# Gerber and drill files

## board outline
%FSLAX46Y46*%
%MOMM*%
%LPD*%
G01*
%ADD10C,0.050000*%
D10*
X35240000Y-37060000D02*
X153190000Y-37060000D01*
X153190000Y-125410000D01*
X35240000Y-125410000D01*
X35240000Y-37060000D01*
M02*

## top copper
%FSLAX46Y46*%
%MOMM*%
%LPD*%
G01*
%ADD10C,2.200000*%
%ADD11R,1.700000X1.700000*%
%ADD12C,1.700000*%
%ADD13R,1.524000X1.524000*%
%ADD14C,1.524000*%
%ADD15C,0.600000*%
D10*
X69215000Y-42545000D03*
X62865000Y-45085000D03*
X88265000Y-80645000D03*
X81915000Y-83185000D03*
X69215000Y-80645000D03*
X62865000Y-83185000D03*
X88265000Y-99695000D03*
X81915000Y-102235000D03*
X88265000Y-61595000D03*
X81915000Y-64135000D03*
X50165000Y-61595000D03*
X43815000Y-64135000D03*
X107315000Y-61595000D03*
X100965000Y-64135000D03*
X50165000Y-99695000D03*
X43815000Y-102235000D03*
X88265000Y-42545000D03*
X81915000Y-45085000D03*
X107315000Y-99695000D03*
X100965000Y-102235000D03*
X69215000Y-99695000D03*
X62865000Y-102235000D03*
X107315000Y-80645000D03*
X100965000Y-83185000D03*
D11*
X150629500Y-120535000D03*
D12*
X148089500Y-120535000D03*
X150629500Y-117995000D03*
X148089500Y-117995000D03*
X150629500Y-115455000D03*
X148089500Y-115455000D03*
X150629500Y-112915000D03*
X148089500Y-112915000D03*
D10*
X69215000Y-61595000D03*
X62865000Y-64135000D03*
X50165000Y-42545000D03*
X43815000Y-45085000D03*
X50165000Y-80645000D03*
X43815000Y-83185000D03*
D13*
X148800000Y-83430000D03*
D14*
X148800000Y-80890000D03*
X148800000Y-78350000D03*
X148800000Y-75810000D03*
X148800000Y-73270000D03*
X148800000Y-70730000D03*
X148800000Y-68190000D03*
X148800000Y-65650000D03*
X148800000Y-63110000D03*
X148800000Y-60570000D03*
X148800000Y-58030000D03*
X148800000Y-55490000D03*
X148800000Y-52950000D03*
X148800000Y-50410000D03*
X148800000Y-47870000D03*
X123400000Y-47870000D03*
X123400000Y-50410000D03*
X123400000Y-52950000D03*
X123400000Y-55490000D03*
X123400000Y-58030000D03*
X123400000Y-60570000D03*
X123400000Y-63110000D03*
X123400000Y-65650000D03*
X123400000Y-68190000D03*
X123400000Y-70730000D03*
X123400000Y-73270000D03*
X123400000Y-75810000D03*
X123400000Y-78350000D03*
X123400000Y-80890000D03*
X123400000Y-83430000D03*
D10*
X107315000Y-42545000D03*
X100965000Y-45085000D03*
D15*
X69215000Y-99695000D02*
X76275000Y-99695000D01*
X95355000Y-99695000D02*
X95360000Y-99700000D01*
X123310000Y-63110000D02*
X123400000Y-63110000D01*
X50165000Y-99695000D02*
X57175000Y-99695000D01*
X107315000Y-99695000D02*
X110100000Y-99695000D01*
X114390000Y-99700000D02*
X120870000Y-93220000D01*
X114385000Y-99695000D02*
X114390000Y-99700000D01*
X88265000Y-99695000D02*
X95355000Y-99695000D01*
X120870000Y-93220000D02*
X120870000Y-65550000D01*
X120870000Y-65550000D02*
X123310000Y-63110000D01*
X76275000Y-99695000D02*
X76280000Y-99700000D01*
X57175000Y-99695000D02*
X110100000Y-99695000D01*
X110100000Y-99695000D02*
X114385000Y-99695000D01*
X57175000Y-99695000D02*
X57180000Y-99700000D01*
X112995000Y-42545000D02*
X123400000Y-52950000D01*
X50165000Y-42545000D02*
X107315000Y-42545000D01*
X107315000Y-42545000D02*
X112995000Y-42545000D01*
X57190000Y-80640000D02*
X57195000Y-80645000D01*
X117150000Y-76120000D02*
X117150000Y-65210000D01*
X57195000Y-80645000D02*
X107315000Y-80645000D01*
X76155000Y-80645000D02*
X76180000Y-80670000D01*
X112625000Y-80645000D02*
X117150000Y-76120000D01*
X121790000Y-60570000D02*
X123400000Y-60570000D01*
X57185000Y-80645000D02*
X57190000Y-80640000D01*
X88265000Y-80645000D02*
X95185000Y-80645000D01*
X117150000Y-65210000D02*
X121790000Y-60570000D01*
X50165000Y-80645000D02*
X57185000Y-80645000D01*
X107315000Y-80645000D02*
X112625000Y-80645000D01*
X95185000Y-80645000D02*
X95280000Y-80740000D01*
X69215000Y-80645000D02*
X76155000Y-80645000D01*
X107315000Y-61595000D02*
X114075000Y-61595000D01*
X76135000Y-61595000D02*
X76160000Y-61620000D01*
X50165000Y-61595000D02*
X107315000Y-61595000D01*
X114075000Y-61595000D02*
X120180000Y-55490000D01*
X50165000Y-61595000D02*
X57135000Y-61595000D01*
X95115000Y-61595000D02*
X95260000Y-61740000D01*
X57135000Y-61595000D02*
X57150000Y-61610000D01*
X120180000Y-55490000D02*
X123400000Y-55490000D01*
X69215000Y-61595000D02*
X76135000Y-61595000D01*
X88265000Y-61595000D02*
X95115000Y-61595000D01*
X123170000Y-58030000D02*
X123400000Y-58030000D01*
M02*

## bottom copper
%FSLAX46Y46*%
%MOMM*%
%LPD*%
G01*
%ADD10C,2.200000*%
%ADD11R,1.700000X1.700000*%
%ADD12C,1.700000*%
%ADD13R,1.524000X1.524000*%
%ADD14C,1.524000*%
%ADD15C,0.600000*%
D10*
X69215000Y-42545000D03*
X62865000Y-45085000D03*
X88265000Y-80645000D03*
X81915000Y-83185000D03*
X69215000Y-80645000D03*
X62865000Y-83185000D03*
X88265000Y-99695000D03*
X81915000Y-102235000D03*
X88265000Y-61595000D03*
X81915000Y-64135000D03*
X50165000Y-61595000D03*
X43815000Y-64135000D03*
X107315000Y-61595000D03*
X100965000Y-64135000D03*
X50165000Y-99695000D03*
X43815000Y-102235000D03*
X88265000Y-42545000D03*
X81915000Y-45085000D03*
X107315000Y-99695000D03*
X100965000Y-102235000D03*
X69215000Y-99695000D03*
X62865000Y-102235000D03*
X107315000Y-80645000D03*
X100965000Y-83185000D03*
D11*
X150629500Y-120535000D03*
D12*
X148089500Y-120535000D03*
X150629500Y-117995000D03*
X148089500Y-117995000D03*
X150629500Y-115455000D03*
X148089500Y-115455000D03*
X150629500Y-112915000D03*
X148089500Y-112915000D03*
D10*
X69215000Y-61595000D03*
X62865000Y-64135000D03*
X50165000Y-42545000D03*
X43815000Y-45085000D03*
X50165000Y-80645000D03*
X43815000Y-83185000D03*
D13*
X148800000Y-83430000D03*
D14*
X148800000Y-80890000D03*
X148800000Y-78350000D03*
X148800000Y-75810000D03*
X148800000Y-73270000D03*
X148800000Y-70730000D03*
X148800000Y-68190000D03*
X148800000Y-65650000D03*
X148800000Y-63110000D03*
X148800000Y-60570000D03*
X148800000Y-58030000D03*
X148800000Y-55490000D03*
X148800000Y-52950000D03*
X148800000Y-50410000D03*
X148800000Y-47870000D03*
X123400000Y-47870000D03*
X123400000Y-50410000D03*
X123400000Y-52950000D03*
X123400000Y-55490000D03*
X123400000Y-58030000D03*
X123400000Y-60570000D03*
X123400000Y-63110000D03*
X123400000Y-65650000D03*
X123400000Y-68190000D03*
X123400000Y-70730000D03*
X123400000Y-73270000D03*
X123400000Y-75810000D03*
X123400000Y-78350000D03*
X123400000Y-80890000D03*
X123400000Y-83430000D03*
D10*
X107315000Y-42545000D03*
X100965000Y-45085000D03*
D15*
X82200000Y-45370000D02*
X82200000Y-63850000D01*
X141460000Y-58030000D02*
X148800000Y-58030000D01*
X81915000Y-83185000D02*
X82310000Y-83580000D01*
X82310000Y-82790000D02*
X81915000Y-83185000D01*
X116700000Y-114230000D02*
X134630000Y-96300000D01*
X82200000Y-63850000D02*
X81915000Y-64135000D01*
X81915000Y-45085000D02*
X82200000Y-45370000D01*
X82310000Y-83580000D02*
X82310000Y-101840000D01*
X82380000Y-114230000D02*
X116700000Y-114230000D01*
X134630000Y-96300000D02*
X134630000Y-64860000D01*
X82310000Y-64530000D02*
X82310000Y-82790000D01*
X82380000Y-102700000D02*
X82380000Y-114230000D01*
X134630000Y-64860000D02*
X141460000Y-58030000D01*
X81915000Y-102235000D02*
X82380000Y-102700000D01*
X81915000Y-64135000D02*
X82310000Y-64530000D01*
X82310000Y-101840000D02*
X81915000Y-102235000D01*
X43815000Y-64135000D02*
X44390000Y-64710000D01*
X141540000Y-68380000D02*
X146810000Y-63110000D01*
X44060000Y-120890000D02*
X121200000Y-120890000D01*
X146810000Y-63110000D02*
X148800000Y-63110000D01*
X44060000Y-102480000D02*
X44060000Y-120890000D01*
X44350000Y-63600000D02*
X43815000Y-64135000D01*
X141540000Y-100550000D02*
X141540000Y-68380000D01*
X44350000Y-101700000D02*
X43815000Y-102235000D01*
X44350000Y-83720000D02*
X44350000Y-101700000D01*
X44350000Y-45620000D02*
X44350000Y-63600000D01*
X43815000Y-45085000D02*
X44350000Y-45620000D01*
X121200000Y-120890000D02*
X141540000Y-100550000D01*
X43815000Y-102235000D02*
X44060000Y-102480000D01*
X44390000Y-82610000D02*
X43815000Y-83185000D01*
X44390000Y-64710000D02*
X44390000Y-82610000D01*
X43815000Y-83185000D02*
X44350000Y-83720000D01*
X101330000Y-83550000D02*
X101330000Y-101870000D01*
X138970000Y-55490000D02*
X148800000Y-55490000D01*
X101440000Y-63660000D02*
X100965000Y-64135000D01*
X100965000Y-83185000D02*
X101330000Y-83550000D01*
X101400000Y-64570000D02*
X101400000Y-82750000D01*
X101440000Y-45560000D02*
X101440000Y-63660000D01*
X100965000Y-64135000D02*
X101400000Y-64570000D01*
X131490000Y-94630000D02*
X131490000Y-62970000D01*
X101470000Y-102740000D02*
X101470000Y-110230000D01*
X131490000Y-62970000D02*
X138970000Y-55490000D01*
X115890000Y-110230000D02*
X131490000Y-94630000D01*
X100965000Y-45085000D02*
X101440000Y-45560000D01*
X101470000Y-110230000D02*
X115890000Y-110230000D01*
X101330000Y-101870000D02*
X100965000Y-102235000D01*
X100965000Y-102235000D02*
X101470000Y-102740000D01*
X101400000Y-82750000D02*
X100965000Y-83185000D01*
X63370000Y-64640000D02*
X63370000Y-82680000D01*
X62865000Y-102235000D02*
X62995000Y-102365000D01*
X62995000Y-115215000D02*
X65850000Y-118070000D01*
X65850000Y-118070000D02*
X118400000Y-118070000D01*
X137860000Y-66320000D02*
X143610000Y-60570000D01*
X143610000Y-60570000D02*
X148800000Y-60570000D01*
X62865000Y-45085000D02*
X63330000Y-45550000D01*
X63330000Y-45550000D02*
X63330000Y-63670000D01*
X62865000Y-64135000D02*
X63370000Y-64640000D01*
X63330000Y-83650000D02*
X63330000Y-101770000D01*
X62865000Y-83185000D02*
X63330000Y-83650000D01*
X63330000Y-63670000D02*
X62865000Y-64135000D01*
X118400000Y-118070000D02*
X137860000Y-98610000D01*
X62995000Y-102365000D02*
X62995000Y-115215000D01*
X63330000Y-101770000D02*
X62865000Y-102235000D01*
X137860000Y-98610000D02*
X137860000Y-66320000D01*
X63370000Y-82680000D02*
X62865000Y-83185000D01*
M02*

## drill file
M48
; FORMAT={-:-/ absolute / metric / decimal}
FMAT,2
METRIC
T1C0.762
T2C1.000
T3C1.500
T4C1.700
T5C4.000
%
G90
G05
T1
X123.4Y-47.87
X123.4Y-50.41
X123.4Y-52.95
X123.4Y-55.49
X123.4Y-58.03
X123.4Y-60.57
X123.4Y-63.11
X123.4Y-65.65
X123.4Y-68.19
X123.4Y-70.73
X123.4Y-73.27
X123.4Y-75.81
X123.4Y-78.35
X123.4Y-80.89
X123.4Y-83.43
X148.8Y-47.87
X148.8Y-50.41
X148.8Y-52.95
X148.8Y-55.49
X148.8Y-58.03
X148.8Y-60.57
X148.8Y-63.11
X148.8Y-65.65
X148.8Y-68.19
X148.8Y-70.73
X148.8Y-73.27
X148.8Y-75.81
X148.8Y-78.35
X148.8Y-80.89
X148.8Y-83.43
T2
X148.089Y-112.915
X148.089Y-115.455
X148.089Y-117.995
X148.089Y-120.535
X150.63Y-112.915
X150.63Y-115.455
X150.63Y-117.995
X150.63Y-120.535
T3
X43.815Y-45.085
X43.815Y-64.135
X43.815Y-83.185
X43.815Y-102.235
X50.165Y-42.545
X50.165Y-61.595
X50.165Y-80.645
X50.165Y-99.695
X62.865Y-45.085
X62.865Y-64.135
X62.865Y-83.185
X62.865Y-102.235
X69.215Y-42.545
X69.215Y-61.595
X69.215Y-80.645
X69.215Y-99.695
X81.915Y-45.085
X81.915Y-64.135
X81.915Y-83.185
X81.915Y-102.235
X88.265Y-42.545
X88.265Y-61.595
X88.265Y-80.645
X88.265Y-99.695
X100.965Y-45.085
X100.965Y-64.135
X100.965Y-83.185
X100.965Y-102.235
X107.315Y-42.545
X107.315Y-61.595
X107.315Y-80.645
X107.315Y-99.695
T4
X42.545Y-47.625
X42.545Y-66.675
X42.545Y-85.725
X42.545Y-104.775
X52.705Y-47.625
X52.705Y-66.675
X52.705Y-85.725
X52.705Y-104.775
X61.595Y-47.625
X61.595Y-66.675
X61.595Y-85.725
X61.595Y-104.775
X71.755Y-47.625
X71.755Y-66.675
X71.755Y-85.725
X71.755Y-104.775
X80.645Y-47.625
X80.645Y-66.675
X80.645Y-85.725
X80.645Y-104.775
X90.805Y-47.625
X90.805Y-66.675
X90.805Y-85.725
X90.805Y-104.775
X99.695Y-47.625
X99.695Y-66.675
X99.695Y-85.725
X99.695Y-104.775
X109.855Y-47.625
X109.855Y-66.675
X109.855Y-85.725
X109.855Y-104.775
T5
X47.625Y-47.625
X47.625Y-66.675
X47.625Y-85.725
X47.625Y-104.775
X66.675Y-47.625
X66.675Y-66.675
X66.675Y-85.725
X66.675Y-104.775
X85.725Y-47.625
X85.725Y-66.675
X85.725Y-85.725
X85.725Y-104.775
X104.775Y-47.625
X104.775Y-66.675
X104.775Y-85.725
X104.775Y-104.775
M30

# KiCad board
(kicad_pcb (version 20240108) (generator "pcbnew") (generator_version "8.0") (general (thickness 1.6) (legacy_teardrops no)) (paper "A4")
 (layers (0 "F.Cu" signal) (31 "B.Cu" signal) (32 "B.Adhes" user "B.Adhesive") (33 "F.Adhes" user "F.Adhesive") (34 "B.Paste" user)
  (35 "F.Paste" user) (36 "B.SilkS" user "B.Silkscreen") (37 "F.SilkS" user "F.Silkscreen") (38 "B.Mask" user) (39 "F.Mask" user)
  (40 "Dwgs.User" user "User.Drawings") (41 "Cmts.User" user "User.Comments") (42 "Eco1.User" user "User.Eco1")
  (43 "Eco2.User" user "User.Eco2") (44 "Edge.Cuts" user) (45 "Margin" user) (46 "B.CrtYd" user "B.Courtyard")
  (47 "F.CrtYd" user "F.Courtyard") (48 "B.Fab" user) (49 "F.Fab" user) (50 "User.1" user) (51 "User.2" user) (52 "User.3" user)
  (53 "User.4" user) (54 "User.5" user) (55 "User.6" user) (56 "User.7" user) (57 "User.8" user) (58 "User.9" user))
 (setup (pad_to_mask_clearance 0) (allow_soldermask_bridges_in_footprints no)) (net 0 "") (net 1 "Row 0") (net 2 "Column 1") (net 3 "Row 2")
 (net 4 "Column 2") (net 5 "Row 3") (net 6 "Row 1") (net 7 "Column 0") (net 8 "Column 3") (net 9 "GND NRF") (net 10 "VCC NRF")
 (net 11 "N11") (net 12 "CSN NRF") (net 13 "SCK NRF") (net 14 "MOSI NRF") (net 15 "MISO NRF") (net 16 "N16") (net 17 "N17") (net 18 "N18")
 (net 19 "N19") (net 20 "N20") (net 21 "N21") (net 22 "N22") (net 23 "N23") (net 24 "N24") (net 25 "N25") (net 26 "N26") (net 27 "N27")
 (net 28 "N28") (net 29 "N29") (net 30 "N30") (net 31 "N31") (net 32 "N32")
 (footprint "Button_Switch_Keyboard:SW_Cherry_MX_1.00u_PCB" (layer "F.Cu") (at 69.215 42.545)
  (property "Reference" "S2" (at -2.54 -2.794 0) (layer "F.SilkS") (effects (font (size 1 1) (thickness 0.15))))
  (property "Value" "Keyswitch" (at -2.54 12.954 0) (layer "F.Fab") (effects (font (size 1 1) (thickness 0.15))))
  (pad "" np_thru_hole circle (at -7.62 5.08) (size 1.7 1.7) (drill 1.7) (layers "*.Cu" "*.Mask"))
  (pad "" np_thru_hole circle (at -2.54 5.08) (size 4 4) (drill 4) (layers "*.Cu" "*.Mask"))
  (pad "" np_thru_hole circle (at 2.54 5.08) (size 1.7 1.7) (drill 1.7) (layers "*.Cu" "*.Mask"))
  (pad "1" thru_hole circle (at 0 0) (size 2.2 2.2) (drill 1.5) (layers "*.Cu" "*.Mask") (remove_unused_layers no) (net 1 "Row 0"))
  (pad "2" thru_hole circle (at -6.35 2.54) (size 2.2 2.2) (drill 1.5) (layers "*.Cu" "*.Mask") (remove_unused_layers no) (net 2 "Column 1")))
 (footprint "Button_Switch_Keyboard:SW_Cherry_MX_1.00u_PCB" (layer "F.Cu") (at 88.265 80.645)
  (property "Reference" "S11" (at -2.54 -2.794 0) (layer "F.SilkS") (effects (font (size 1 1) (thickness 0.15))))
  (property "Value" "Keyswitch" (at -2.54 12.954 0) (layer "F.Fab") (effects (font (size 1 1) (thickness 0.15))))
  (pad "" np_thru_hole circle (at -7.62 5.08) (size 1.7 1.7) (drill 1.7) (layers "*.Cu" "*.Mask"))
  (pad "" np_thru_hole circle (at -2.54 5.08) (size 4 4) (drill 4) (layers "*.Cu" "*.Mask"))
  (pad "" np_thru_hole circle (at 2.54 5.08) (size 1.7 1.7) (drill 1.7) (layers "*.Cu" "*.Mask"))
  (pad "1" thru_hole circle (at 0 0) (size 2.2 2.2) (drill 1.5) (layers "*.Cu" "*.Mask") (remove_unused_layers no) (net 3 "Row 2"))
  (pad "2" thru_hole circle (at -6.35 2.54) (size 2.2 2.2) (drill 1.5) (layers "*.Cu" "*.Mask") (remove_unused_layers no) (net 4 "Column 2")))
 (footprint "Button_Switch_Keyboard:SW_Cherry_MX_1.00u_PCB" (layer "F.Cu") (at 69.215 80.645)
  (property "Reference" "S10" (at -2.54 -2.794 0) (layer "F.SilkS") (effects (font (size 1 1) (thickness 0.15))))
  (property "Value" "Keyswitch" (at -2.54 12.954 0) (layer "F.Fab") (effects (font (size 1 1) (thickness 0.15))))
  (pad "" np_thru_hole circle (at -7.62 5.08) (size 1.7 1.7) (drill 1.7) (layers "*.Cu" "*.Mask"))
  (pad "" np_thru_hole circle (at -2.54 5.08) (size 4 4) (drill 4) (layers "*.Cu" "*.Mask"))
  (pad "" np_thru_hole circle (at 2.54 5.08) (size 1.7 1.7) (drill 1.7) (layers "*.Cu" "*.Mask"))
  (pad "1" thru_hole circle (at 0 0) (size 2.2 2.2) (drill 1.5) (layers "*.Cu" "*.Mask") (remove_unused_layers no) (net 3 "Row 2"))
  (pad "2" thru_hole circle (at -6.35 2.54) (size 2.2 2.2) (drill 1.5) (layers "*.Cu" "*.Mask") (remove_unused_layers no) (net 2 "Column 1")))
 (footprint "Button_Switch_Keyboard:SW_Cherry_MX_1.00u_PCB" (layer "F.Cu") (at 88.265 99.695)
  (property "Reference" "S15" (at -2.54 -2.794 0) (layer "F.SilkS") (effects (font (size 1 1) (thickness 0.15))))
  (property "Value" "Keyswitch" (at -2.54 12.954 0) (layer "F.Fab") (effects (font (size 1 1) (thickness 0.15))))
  (pad "" np_thru_hole circle (at -7.62 5.08) (size 1.7 1.7) (drill 1.7) (layers "*.Cu" "*.Mask"))
  (pad "" np_thru_hole circle (at -2.54 5.08) (size 4 4) (drill 4) (layers "*.Cu" "*.Mask"))
  (pad "" np_thru_hole circle (at 2.54 5.08) (size 1.7 1.7) (drill 1.7) (layers "*.Cu" "*.Mask"))
  (pad "1" thru_hole circle (at 0 0) (size 2.2 2.2) (drill 1.5) (layers "*.Cu" "*.Mask") (remove_unused_layers no) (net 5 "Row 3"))
  (pad "2" thru_hole circle (at -6.35 2.54) (size 2.2 2.2) (drill 1.5) (layers "*.Cu" "*.Mask") (remove_unused_layers no) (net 4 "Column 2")))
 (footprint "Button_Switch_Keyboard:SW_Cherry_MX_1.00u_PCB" (layer "F.Cu") (at 88.265 61.595)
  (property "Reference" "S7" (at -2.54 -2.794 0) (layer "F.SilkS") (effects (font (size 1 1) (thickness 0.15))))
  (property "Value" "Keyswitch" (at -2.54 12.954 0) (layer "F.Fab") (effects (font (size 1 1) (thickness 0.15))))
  (pad "" np_thru_hole circle (at -7.62 5.08) (size 1.7 1.7) (drill 1.7) (layers "*.Cu" "*.Mask"))
  (pad "" np_thru_hole circle (at -2.54 5.08) (size 4 4) (drill 4) (layers "*.Cu" "*.Mask"))
  (pad "" np_thru_hole circle (at 2.54 5.08) (size 1.7 1.7) (drill 1.7) (layers "*.Cu" "*.Mask"))
  (pad "1" thru_hole circle (at 0 0) (size 2.2 2.2) (drill 1.5) (layers "*.Cu" "*.Mask") (remove_unused_layers no) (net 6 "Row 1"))
  (pad "2" thru_hole circle (at -6.35 2.54) (size 2.2 2.2) (drill 1.5) (layers "*.Cu" "*.Mask") (remove_unused_layers no) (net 4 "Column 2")))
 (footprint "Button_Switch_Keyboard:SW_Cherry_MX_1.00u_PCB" (layer "F.Cu") (at 50.165 61.595)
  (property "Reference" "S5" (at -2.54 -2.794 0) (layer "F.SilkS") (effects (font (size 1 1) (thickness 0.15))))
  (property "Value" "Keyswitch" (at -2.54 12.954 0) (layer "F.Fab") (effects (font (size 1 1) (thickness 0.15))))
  (pad "" np_thru_hole circle (at -7.62 5.08) (size 1.7 1.7) (drill 1.7) (layers "*.Cu" "*.Mask"))
  (pad "" np_thru_hole circle (at -2.54 5.08) (size 4 4) (drill 4) (layers "*.Cu" "*.Mask"))
  (pad "" np_thru_hole circle (at 2.54 5.08) (size 1.7 1.7) (drill 1.7) (layers "*.Cu" "*.Mask"))
  (pad "1" thru_hole circle (at 0 0) (size 2.2 2.2) (drill 1.5) (layers "*.Cu" "*.Mask") (remove_unused_layers no) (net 6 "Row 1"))
  (pad "2" thru_hole circle (at -6.35 2.54) (size 2.2 2.2) (drill 1.5) (layers "*.Cu" "*.Mask") (remove_unused_layers no) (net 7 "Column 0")))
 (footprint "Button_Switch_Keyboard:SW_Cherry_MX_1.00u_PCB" (layer "F.Cu") (at 107.315 61.595)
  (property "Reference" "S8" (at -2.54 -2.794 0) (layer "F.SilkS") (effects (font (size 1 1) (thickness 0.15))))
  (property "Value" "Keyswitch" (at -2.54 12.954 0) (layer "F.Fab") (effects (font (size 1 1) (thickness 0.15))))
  (pad "" np_thru_hole circle (at -7.62 5.08) (size 1.7 1.7) (drill 1.7) (layers "*.Cu" "*.Mask"))
  (pad "" np_thru_hole circle (at -2.54 5.08) (size 4 4) (drill 4) (layers "*.Cu" "*.Mask"))
  (pad "" np_thru_hole circle (at 2.54 5.08) (size 1.7 1.7) (drill 1.7) (layers "*.Cu" "*.Mask"))
  (pad "1" thru_hole circle (at 0 0) (size 2.2 2.2) (drill 1.5) (layers "*.Cu" "*.Mask") (remove_unused_layers no) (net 6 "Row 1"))
  (pad "2" thru_hole circle (at -6.35 2.54) (size 2.2 2.2) (drill 1.5) (layers "*.Cu" "*.Mask") (remove_unused_layers no) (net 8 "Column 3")))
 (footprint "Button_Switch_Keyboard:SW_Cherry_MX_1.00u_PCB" (layer "F.Cu") (at 50.165 99.695)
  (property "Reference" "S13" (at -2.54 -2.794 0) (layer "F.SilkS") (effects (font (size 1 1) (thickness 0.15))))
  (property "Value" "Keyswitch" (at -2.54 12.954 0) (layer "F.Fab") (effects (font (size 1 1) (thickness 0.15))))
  (pad "" np_thru_hole circle (at -7.62 5.08) (size 1.7 1.7) (drill 1.7) (layers "*.Cu" "*.Mask"))
  (pad "" np_thru_hole circle (at -2.54 5.08) (size 4 4) (drill 4) (layers "*.Cu" "*.Mask"))
  (pad "" np_thru_hole circle (at 2.54 5.08) (size 1.7 1.7) (drill 1.7) (layers "*.Cu" "*.Mask"))
  (pad "1" thru_hole circle (at 0 0) (size 2.2 2.2) (drill 1.5) (layers "*.Cu" "*.Mask") (remove_unused_layers no) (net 5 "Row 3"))
  (pad "2" thru_hole circle (at -6.35 2.54) (size 2.2 2.2) (drill 1.5) (layers "*.Cu" "*.Mask") (remove_unused_layers no) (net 7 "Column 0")))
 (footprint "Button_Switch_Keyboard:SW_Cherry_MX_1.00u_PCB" (layer "F.Cu") (at 88.265 42.545)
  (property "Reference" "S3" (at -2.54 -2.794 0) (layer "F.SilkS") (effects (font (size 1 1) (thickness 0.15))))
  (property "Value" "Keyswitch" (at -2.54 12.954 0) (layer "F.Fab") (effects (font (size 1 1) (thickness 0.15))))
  (pad "" np_thru_hole circle (at -7.62 5.08) (size 1.7 1.7) (drill 1.7) (layers "*.Cu" "*.Mask"))
  (pad "" np_thru_hole circle (at -2.54 5.08) (size 4 4) (drill 4) (layers "*.Cu" "*.Mask"))
  (pad "" np_thru_hole circle (at 2.54 5.08) (size 1.7 1.7) (drill 1.7) (layers "*.Cu" "*.Mask"))
  (pad "1" thru_hole circle (at 0 0) (size 2.2 2.2) (drill 1.5) (layers "*.Cu" "*.Mask") (remove_unused_layers no) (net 1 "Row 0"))
  (pad "2" thru_hole circle (at -6.35 2.54) (size 2.2 2.2) (drill 1.5) (layers "*.Cu" "*.Mask") (remove_unused_layers no) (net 4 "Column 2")))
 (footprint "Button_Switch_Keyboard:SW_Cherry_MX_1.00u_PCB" (layer "F.Cu") (at 107.315 99.695)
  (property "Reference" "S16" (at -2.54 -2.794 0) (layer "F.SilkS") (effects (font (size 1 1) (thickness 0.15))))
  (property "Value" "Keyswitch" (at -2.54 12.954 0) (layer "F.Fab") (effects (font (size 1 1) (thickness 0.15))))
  (pad "" np_thru_hole circle (at -7.62 5.08) (size 1.7 1.7) (drill 1.7) (layers "*.Cu" "*.Mask"))
  (pad "" np_thru_hole circle (at -2.54 5.08) (size 4 4) (drill 4) (layers "*.Cu" "*.Mask"))
  (pad "" np_thru_hole circle (at 2.54 5.08) (size 1.7 1.7) (drill 1.7) (layers "*.Cu" "*.Mask"))
  (pad "1" thru_hole circle (at 0 0) (size 2.2 2.2) (drill 1.5) (layers "*.Cu" "*.Mask") (remove_unused_layers no) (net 5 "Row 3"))
  (pad "2" thru_hole circle (at -6.35 2.54) (size 2.2 2.2) (drill 1.5) (layers "*.Cu" "*.Mask") (remove_unused_layers no) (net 8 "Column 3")))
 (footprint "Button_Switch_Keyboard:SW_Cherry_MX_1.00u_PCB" (layer "F.Cu") (at 69.215 99.695)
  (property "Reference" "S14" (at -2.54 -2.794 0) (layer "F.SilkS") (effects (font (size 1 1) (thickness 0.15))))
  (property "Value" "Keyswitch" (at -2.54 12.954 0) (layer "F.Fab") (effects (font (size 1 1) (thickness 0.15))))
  (pad "" np_thru_hole circle (at -7.62 5.08) (size 1.7 1.7) (drill 1.7) (layers "*.Cu" "*.Mask"))
  (pad "" np_thru_hole circle (at -2.54 5.08) (size 4 4) (drill 4) (layers "*.Cu" "*.Mask"))
  (pad "" np_thru_hole circle (at 2.54 5.08) (size 1.7 1.7) (drill 1.7) (layers "*.Cu" "*.Mask"))
  (pad "1" thru_hole circle (at 0 0) (size 2.2 2.2) (drill 1.5) (layers "*.Cu" "*.Mask") (remove_unused_layers no) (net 5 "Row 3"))
  (pad "2" thru_hole circle (at -6.35 2.54) (size 2.2 2.2) (drill 1.5) (layers "*.Cu" "*.Mask") (remove_unused_layers no) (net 2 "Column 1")))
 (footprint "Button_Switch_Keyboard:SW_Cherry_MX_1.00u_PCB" (layer "F.Cu") (at 107.315 80.645)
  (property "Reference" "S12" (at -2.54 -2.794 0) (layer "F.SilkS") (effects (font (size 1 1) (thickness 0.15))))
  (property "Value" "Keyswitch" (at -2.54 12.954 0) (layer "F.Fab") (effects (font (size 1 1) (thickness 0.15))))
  (pad "" np_thru_hole circle (at -7.62 5.08) (size 1.7 1.7) (drill 1.7) (layers "*.Cu" "*.Mask"))
  (pad "" np_thru_hole circle (at -2.54 5.08) (size 4 4) (drill 4) (layers "*.Cu" "*.Mask"))
  (pad "" np_thru_hole circle (at 2.54 5.08) (size 1.7 1.7) (drill 1.7) (layers "*.Cu" "*.Mask"))
  (pad "1" thru_hole circle (at 0 0) (size 2.2 2.2) (drill 1.5) (layers "*.Cu" "*.Mask") (remove_unused_layers no) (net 3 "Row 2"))
  (pad "2" thru_hole circle (at -6.35 2.54) (size 2.2 2.2) (drill 1.5) (layers "*.Cu" "*.Mask") (remove_unused_layers no) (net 8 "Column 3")))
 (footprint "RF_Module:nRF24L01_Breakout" (layer "F.Cu") (at 150.6295 120.535 180)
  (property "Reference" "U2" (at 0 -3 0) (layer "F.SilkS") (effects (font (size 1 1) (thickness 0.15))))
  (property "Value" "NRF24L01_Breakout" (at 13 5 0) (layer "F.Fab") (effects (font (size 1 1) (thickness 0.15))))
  (pad "1" thru_hole rect (at 0 0 180) (size 1.7 1.7) (drill 1) (layers "*.Cu" "*.Mask") (remove_unused_layers no) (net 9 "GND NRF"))
  (pad "2" thru_hole circle (at 2.54 0 180) (size 1.7 1.7) (drill 1) (layers "*.Cu" "*.Mask") (remove_unused_layers no) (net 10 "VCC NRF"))
  (pad "3" thru_hole circle (at 0 2.54 180) (size 1.7 1.7) (drill 1) (layers "*.Cu" "*.Mask") (remove_unused_layers no) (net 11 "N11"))
  (pad "4" thru_hole circle (at 2.54 2.54 180) (size 1.7 1.7) (drill 1) (layers "*.Cu" "*.Mask") (remove_unused_layers no)
   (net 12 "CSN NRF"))
  (pad "5" thru_hole circle (at 0 5.08 180) (size 1.7 1.7) (drill 1) (layers "*.Cu" "*.Mask") (remove_unused_layers no) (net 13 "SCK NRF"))
  (pad "6" thru_hole circle (at 2.54 5.08 180) (size 1.7 1.7) (drill 1) (layers "*.Cu" "*.Mask") (remove_unused_layers no)
   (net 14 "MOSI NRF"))
  (pad "7" thru_hole circle (at 0 7.62 180) (size 1.7 1.7) (drill 1) (layers "*.Cu" "*.Mask") (remove_unused_layers no) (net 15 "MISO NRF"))
  (pad "8" thru_hole circle (at 2.54 7.62 180) (size 1.7 1.7) (drill 1) (layers "*.Cu" "*.Mask") (remove_unused_layers no) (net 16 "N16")))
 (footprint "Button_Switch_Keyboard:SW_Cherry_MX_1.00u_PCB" (layer "F.Cu") (at 69.215 61.595)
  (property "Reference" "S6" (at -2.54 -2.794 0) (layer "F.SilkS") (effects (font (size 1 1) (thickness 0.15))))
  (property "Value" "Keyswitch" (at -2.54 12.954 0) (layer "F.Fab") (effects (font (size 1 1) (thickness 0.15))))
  (pad "" np_thru_hole circle (at -7.62 5.08) (size 1.7 1.7) (drill 1.7) (layers "*.Cu" "*.Mask"))
  (pad "" np_thru_hole circle (at -2.54 5.08) (size 4 4) (drill 4) (layers "*.Cu" "*.Mask"))
  (pad "" np_thru_hole circle (at 2.54 5.08) (size 1.7 1.7) (drill 1.7) (layers "*.Cu" "*.Mask"))
  (pad "1" thru_hole circle (at 0 0) (size 2.2 2.2) (drill 1.5) (layers "*.Cu" "*.Mask") (remove_unused_layers no) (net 6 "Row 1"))
  (pad "2" thru_hole circle (at -6.35 2.54) (size 2.2 2.2) (drill 1.5) (layers "*.Cu" "*.Mask") (remove_unused_layers no) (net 2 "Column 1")))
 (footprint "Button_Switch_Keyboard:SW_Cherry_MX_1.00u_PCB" (layer "F.Cu") (at 50.165 42.545)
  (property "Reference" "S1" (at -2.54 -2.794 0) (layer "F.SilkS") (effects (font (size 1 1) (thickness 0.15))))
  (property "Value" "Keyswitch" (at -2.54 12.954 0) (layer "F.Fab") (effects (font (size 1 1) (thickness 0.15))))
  (pad "" np_thru_hole circle (at -7.62 5.08) (size 1.7 1.7) (drill 1.7) (layers "*.Cu" "*.Mask"))
  (pad "" np_thru_hole circle (at -2.54 5.08) (size 4 4) (drill 4) (layers "*.Cu" "*.Mask"))
  (pad "" np_thru_hole circle (at 2.54 5.08) (size 1.7 1.7) (drill 1.7) (layers "*.Cu" "*.Mask"))
  (pad "1" thru_hole circle (at 0 0) (size 2.2 2.2) (drill 1.5) (layers "*.Cu" "*.Mask") (remove_unused_layers no) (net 1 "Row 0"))
  (pad "2" thru_hole circle (at -6.35 2.54) (size 2.2 2.2) (drill 1.5) (layers "*.Cu" "*.Mask") (remove_unused_layers no) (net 7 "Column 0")))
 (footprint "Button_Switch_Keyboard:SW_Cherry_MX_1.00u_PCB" (layer "F.Cu") (at 50.165 80.645)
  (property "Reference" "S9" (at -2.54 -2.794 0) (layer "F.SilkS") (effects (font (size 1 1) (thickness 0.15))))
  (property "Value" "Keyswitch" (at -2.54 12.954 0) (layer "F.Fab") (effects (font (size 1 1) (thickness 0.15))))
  (pad "" np_thru_hole circle (at -7.62 5.08) (size 1.7 1.7) (drill 1.7) (layers "*.Cu" "*.Mask"))
  (pad "" np_thru_hole circle (at -2.54 5.08) (size 4 4) (drill 4) (layers "*.Cu" "*.Mask"))
  (pad "" np_thru_hole circle (at 2.54 5.08) (size 1.7 1.7) (drill 1.7) (layers "*.Cu" "*.Mask"))
  (pad "1" thru_hole circle (at 0 0) (size 2.2 2.2) (drill 1.5) (layers "*.Cu" "*.Mask") (remove_unused_layers no) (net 3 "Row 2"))
  (pad "2" thru_hole circle (at -6.35 2.54) (size 2.2 2.2) (drill 1.5) (layers "*.Cu" "*.Mask") (remove_unused_layers no) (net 7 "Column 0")))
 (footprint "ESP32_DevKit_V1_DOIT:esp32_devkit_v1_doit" (layer "F.Cu") (at 136.1 83.43 180)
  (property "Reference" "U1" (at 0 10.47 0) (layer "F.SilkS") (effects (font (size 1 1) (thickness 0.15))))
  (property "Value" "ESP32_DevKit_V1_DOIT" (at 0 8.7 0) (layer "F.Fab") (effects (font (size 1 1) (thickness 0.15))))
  (pad "1" thru_hole rect (at -12.7 0 180) (size 1.524 1.524) (drill 0.762) (layers "*.Cu" "*.Mask") (remove_unused_layers no)
   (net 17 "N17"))
  (pad "2" thru_hole circle (at -12.7 2.54 180) (size 1.524 1.524) (drill 0.762) (layers "*.Cu" "*.Mask") (remove_unused_layers no)
   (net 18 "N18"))
  (pad "3" thru_hole circle (at -12.7 5.08 180) (size 1.524 1.524) (drill 0.762) (layers "*.Cu" "*.Mask") (remove_unused_layers no)
   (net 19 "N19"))
  (pad "4" thru_hole circle (at -12.7 7.62 180) (size 1.524 1.524) (drill 0.762) (layers "*.Cu" "*.Mask") (remove_unused_layers no)
   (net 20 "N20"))
  (pad "5" thru_hole circle (at -12.7 10.16 180) (size 1.524 1.524) (drill 0.762) (layers "*.Cu" "*.Mask") (remove_unused_layers no)
   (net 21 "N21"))
  (pad "6" thru_hole circle (at -12.7 12.7 180) (size 1.524 1.524) (drill 0.762) (layers "*.Cu" "*.Mask") (remove_unused_layers no)
   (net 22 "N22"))
  (pad "7" thru_hole circle (at -12.7 15.24 180) (size 1.524 1.524) (drill 0.762) (layers "*.Cu" "*.Mask") (remove_unused_layers no)
   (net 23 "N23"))
  (pad "8" thru_hole circle (at -12.7 17.78 180) (size 1.524 1.524) (drill 0.762) (layers "*.Cu" "*.Mask") (remove_unused_layers no)
   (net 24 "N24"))
  (pad "9" thru_hole circle (at -12.7 20.32 180) (size 1.524 1.524) (drill 0.762) (layers "*.Cu" "*.Mask") (remove_unused_layers no)
   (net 7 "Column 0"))
  (pad "10" thru_hole circle (at -12.7 22.86 180) (size 1.524 1.524) (drill 0.762) (layers "*.Cu" "*.Mask") (remove_unused_layers no)
   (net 2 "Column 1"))
  (pad "11" thru_hole circle (at -12.7 25.4 180) (size 1.524 1.524) (drill 0.762) (layers "*.Cu" "*.Mask") (remove_unused_layers no)
   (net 4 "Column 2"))
  (pad "12" thru_hole circle (at -12.7 27.94 180) (size 1.524 1.524) (drill 0.762) (layers "*.Cu" "*.Mask") (remove_unused_layers no)
   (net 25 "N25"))
  (pad "13" thru_hole circle (at -12.7 30.48 180) (size 1.524 1.524) (drill 0.762) (layers "*.Cu" "*.Mask") (remove_unused_layers no)
   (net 8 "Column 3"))
  (pad "14" thru_hole circle (at -12.7 33.02 180) (size 1.524 1.524) (drill 0.762) (layers "*.Cu" "*.Mask") (remove_unused_layers no)
   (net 9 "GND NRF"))
  (pad "15" thru_hole circle (at -12.7 35.56 180) (size 1.524 1.524) (drill 0.762) (layers "*.Cu" "*.Mask") (remove_unused_layers no)
   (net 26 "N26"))
  (pad "16" thru_hole circle (at 12.7 35.56 180) (size 1.524 1.524) (drill 0.762) (layers "*.Cu" "*.Mask") (remove_unused_layers no)
   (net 10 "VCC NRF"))
  (pad "17" thru_hole circle (at 12.7 33.02 180) (size 1.524 1.524) (drill 0.762) (layers "*.Cu" "*.Mask") (remove_unused_layers no)
   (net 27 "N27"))
  (pad "18" thru_hole circle (at 12.7 30.48 180) (size 1.524 1.524) (drill 0.762) (layers "*.Cu" "*.Mask") (remove_unused_layers no)
   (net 1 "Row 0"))
  (pad "19" thru_hole circle (at 12.7 27.94 180) (size 1.524 1.524) (drill 0.762) (layers "*.Cu" "*.Mask") (remove_unused_layers no)
   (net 6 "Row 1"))
  (pad "20" thru_hole circle (at 12.7 25.4 180) (size 1.524 1.524) (drill 0.762) (layers "*.Cu" "*.Mask") (remove_unused_layers no)
   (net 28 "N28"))
  (pad "21" thru_hole circle (at 12.7 22.86 180) (size 1.524 1.524) (drill 0.762) (layers "*.Cu" "*.Mask") (remove_unused_layers no)
   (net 3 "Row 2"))
  (pad "22" thru_hole circle (at 12.7 20.32 180) (size 1.524 1.524) (drill 0.762) (layers "*.Cu" "*.Mask") (remove_unused_layers no)
   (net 5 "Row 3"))
  (pad "23" thru_hole circle (at 12.7 17.78 180) (size 1.524 1.524) (drill 0.762) (layers "*.Cu" "*.Mask") (remove_unused_layers no)
   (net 12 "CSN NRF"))
  (pad "24" thru_hole circle (at 12.7 15.24 180) (size 1.524 1.524) (drill 0.762) (layers "*.Cu" "*.Mask") (remove_unused_layers no)
   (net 13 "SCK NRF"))
  (pad "25" thru_hole circle (at 12.7 12.7 180) (size 1.524 1.524) (drill 0.762) (layers "*.Cu" "*.Mask") (remove_unused_layers no)
   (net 15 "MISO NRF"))
  (pad "26" thru_hole circle (at 12.7 10.16 180) (size 1.524 1.524) (drill 0.762) (layers "*.Cu" "*.Mask") (remove_unused_layers no)
   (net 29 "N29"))
  (pad "27" thru_hole circle (at 12.7 7.62 180) (size 1.524 1.524) (drill 0.762) (layers "*.Cu" "*.Mask") (remove_unused_layers no)
   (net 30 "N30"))
  (pad "28" thru_hole circle (at 12.7 5.08 180) (size 1.524 1.524) (drill 0.762) (layers "*.Cu" "*.Mask") (remove_unused_layers no)
   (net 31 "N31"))
  (pad "29" thru_hole circle (at 12.7 2.54 180) (size 1.524 1.524) (drill 0.762) (layers "*.Cu" "*.Mask") (remove_unused_layers no)
   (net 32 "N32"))
  (pad "30" thru_hole circle (at 12.7 0 180) (size 1.524 1.524) (drill 0.762) (layers "*.Cu" "*.Mask") (remove_unused_layers no)
   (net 14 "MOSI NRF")))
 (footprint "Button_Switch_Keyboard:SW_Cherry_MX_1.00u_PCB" (layer "F.Cu") (at 107.315 42.545)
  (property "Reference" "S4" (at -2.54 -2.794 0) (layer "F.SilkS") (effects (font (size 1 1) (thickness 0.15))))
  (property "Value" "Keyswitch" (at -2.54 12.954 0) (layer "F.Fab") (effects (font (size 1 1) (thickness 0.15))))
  (pad "" np_thru_hole circle (at -7.62 5.08) (size 1.7 1.7) (drill 1.7) (layers "*.Cu" "*.Mask"))
  (pad "" np_thru_hole circle (at -2.54 5.08) (size 4 4) (drill 4) (layers "*.Cu" "*.Mask"))
  (pad "" np_thru_hole circle (at 2.54 5.08) (size 1.7 1.7) (drill 1.7) (layers "*.Cu" "*.Mask"))
  (pad "1" thru_hole circle (at 0 0) (size 2.2 2.2) (drill 1.5) (layers "*.Cu" "*.Mask") (remove_unused_layers no) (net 1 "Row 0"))
  (pad "2" thru_hole circle (at -6.35 2.54) (size 2.2 2.2) (drill 1.5) (layers "*.Cu" "*.Mask") (remove_unused_layers no) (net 8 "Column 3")))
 (gr_rect (start 35.24 37.06) (end 153.19 125.41) (stroke (width 0.05) (type default)) (fill none) (layer "Edge.Cuts"))
 (segment (start 69.215 99.695) (end 76.275 99.695) (width 0.6) (layer "F.Cu") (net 5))
 (segment (start 95.355 99.695) (end 95.36 99.7) (width 0.6) (layer "F.Cu") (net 5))
 (segment (start 123.31 63.11) (end 123.4 63.11) (width 0.6) (layer "F.Cu") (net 5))
 (segment (start 50.165 99.695) (end 57.175 99.695) (width 0.6) (layer "F.Cu") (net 5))
 (segment (start 107.315 99.695) (end 110.1 99.695) (width 0.6) (layer "F.Cu") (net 5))
 (segment (start 114.39 99.7) (end 120.87 93.22) (width 0.6) (layer "F.Cu") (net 5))
 (segment (start 114.385 99.695) (end 114.39 99.7) (width 0.6) (layer "F.Cu") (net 5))
 (segment (start 88.265 99.695) (end 95.355 99.695) (width 0.6) (layer "F.Cu") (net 5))
 (segment (start 120.87 93.22) (end 120.87 65.55) (width 0.6) (layer "F.Cu") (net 5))
 (segment (start 120.87 65.55) (end 123.31 63.11) (width 0.6) (layer "F.Cu") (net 5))
 (segment (start 76.275 99.695) (end 76.28 99.7) (width 0.6) (layer "F.Cu") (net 5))
 (segment (start 57.175 99.695) (end 110.1 99.695) (width 0.6) (layer "F.Cu") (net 5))
 (segment (start 110.1 99.695) (end 114.385 99.695) (width 0.6) (layer "F.Cu") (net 5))
 (segment (start 57.175 99.695) (end 57.18 99.7) (width 0.6) (layer "F.Cu") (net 5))
 (segment (start 82.2 45.37) (end 82.2 63.85) (width 0.6) (layer "B.Cu") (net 4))
 (segment (start 141.46 58.03) (end 148.8 58.03) (width 0.6) (layer "B.Cu") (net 4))
 (segment (start 81.915 83.185) (end 82.31 83.58) (width 0.6) (layer "B.Cu") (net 4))
 (segment (start 82.31 82.79) (end 81.915 83.185) (width 0.6) (layer "B.Cu") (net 4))
 (segment (start 116.7 114.23) (end 134.63 96.3) (width 0.6) (layer "B.Cu") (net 4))
 (segment (start 82.2 63.85) (end 81.915 64.135) (width 0.6) (layer "B.Cu") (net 4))
 (segment (start 81.915 45.085) (end 82.2 45.37) (width 0.6) (layer "B.Cu") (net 4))
 (segment (start 82.31 83.58) (end 82.31 101.84) (width 0.6) (layer "B.Cu") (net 4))
 (segment (start 82.38 114.23) (end 116.7 114.23) (width 0.6) (layer "B.Cu") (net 4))
 (segment (start 134.63 96.3) (end 134.63 64.86) (width 0.6) (layer "B.Cu") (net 4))
 (segment (start 82.31 64.53) (end 82.31 82.79) (width 0.6) (layer "B.Cu") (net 4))
 (segment (start 82.38 102.7) (end 82.38 114.23) (width 0.6) (layer "B.Cu") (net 4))
 (segment (start 134.63 64.86) (end 141.46 58.03) (width 0.6) (layer "B.Cu") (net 4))
 (segment (start 81.915 102.235) (end 82.38 102.7) (width 0.6) (layer "B.Cu") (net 4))
 (segment (start 81.915 64.135) (end 82.31 64.53) (width 0.6) (layer "B.Cu") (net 4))
 (segment (start 82.31 101.84) (end 81.915 102.235) (width 0.6) (layer "B.Cu") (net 4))
 (segment (start 43.815 64.135) (end 44.39 64.71) (width 0.6) (layer "B.Cu") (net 7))
 (segment (start 141.54 68.38) (end 146.81 63.11) (width 0.6) (layer "B.Cu") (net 7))
 (segment (start 44.06 120.89) (end 121.2 120.89) (width 0.6) (layer "B.Cu") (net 7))
 (segment (start 146.81 63.11) (end 148.8 63.11) (width 0.6) (layer "B.Cu") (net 7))
 (segment (start 44.06 102.48) (end 44.06 120.89) (width 0.6) (layer "B.Cu") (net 7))
 (segment (start 44.35 63.6) (end 43.815 64.135) (width 0.6) (layer "B.Cu") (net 7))
 (segment (start 141.54 100.55) (end 141.54 68.38) (width 0.6) (layer "B.Cu") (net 7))
 (segment (start 44.35 101.7) (end 43.815 102.235) (width 0.6) (layer "B.Cu") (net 7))
 (segment (start 44.35 83.72) (end 44.35 101.7) (width 0.6) (layer "B.Cu") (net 7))
 (segment (start 44.35 45.62) (end 44.35 63.6) (width 0.6) (layer "B.Cu") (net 7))
 (segment (start 43.815 45.085) (end 44.35 45.62) (width 0.6) (layer "B.Cu") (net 7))
 (segment (start 121.2 120.89) (end 141.54 100.55) (width 0.6) (layer "B.Cu") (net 7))
 (segment (start 43.815 102.235) (end 44.06 102.48) (width 0.6) (layer "B.Cu") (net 7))
 (segment (start 44.39 82.61) (end 43.815 83.185) (width 0.6) (layer "B.Cu") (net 7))
 (segment (start 44.39 64.71) (end 44.39 82.61) (width 0.6) (layer "B.Cu") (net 7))
 (segment (start 43.815 83.185) (end 44.35 83.72) (width 0.6) (layer "B.Cu") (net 7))
 (segment (start 112.995 42.545) (end 123.4 52.95) (width 0.6) (layer "F.Cu") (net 1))
 (segment (start 50.165 42.545) (end 107.315 42.545) (width 0.6) (layer "F.Cu") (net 1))
 (segment (start 107.315 42.545) (end 112.995 42.545) (width 0.6) (layer "F.Cu") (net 1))
 (segment (start 101.33 83.55) (end 101.33 101.87) (width 0.6) (layer "B.Cu") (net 8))
 (segment (start 138.97 55.49) (end 148.8 55.49) (width 0.6) (layer "B.Cu") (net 8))
 (segment (start 101.44 63.66) (end 100.965 64.135) (width 0.6) (layer "B.Cu") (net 8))
 (segment (start 100.965 83.185) (end 101.33 83.55) (width 0.6) (layer "B.Cu") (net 8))
 (segment (start 101.4 64.57) (end 101.4 82.75) (width 0.6) (layer "B.Cu") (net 8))
 (segment (start 101.44 45.56) (end 101.44 63.66) (width 0.6) (layer "B.Cu") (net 8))
 (segment (start 100.965 64.135) (end 101.4 64.57) (width 0.6) (layer "B.Cu") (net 8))
 (segment (start 131.49 94.63) (end 131.49 62.97) (width 0.6) (layer "B.Cu") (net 8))
 (segment (start 101.47 102.74) (end 101.47 110.23) (width 0.6) (layer "B.Cu") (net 8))
 (segment (start 131.49 62.97) (end 138.97 55.49) (width 0.6) (layer "B.Cu") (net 8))
 (segment (start 115.89 110.23) (end 131.49 94.63) (width 0.6) (layer "B.Cu") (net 8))
 (segment (start 100.965 45.085) (end 101.44 45.56) (width 0.6) (layer "B.Cu") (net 8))
 (segment (start 101.47 110.23) (end 115.89 110.23) (width 0.6) (layer "B.Cu") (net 8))
 (segment (start 101.33 101.87) (end 100.965 102.235) (width 0.6) (layer "B.Cu") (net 8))
 (segment (start 100.965 102.235) (end 101.47 102.74) (width 0.6) (layer "B.Cu") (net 8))
 (segment (start 101.4 82.75) (end 100.965 83.185) (width 0.6) (layer "B.Cu") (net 8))
 (segment (start 63.37 64.64) (end 63.37 82.68) (width 0.6) (layer "B.Cu") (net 2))
 (segment (start 62.865 102.235) (end 62.995 102.365) (width 0.6) (layer "B.Cu") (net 2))
 (segment (start 62.995 115.215) (end 65.85 118.07) (width 0.6) (layer "B.Cu") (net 2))
 (segment (start 65.85 118.07) (end 118.4 118.07) (width 0.6) (layer "B.Cu") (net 2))
 (segment (start 137.86 66.32) (end 143.61 60.57) (width 0.6) (layer "B.Cu") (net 2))
 (segment (start 143.61 60.57) (end 148.8 60.57) (width 0.6) (layer "B.Cu") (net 2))
 (segment (start 62.865 45.085) (end 63.33 45.55) (width 0.6) (layer "B.Cu") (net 2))
 (segment (start 63.33 45.55) (end 63.33 63.67) (width 0.6) (layer "B.Cu") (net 2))
 (segment (start 62.865 64.135) (end 63.37 64.64) (width 0.6) (layer "B.Cu") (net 2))
 (segment (start 63.33 83.65) (end 63.33 101.77) (width 0.6) (layer "B.Cu") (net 2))
 (segment (start 62.865 83.185) (end 63.33 83.65) (width 0.6) (layer "B.Cu") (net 2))
 (segment (start 63.33 63.67) (end 62.865 64.135) (width 0.6) (layer "B.Cu") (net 2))
 (segment (start 118.4 118.07) (end 137.86 98.61) (width 0.6) (layer "B.Cu") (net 2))
 (segment (start 62.995 102.365) (end 62.995 115.215) (width 0.6) (layer "B.Cu") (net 2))
 (segment (start 63.33 101.77) (end 62.865 102.235) (width 0.6) (layer "B.Cu") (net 2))
 (segment (start 137.86 98.61) (end 137.86 66.32) (width 0.6) (layer "B.Cu") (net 2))
 (segment (start 63.37 82.68) (end 62.865 83.185) (width 0.6) (layer "B.Cu") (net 2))
 (segment (start 57.19 80.64) (end 57.195 80.645) (width 0.6) (layer "F.Cu") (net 3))
 (segment (start 117.15 76.12) (end 117.15 65.21) (width 0.6) (layer "F.Cu") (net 3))
 (segment (start 57.195 80.645) (end 107.315 80.645) (width 0.6) (layer "F.Cu") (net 3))
 (segment (start 76.155 80.645) (end 76.18 80.67) (width 0.6) (layer "F.Cu") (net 3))
 (segment (start 112.625 80.645) (end 117.15 76.12) (width 0.6) (layer "F.Cu") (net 3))
 (segment (start 121.79 60.57) (end 123.4 60.57) (width 0.6) (layer "F.Cu") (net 3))
 (segment (start 57.185 80.645) (end 57.19 80.64) (width 0.6) (layer "F.Cu") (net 3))
 (segment (start 88.265 80.645) (end 95.185 80.645) (width 0.6) (layer "F.Cu") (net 3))
 (segment (start 117.15 65.21) (end 121.79 60.57) (width 0.6) (layer "F.Cu") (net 3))
 (segment (start 50.165 80.645) (end 57.185 80.645) (width 0.6) (layer "F.Cu") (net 3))
 (segment (start 107.315 80.645) (end 112.625 80.645) (width 0.6) (layer "F.Cu") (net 3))
 (segment (start 95.185 80.645) (end 95.28 80.74) (width 0.6) (layer "F.Cu") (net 3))
 (segment (start 69.215 80.645) (end 76.155 80.645) (width 0.6) (layer "F.Cu") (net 3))
 (segment (start 107.315 61.595) (end 114.075 61.595) (width 0.6) (layer "F.Cu") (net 6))
 (segment (start 76.135 61.595) (end 76.16 61.62) (width 0.6) (layer "F.Cu") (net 6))
 (segment (start 50.165 61.595) (end 107.315 61.595) (width 0.6) (layer "F.Cu") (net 6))
 (segment (start 114.075 61.595) (end 120.18 55.49) (width 0.6) (layer "F.Cu") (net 6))
 (segment (start 50.165 61.595) (end 57.135 61.595) (width 0.6) (layer "F.Cu") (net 6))
 (segment (start 95.115 61.595) (end 95.26 61.74) (width 0.6) (layer "F.Cu") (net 6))
 (segment (start 57.135 61.595) (end 57.15 61.61) (width 0.6) (layer "F.Cu") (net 6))
 (segment (start 120.18 55.49) (end 123.4 55.49) (width 0.6) (layer "F.Cu") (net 6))
 (segment (start 69.215 61.595) (end 76.135 61.595) (width 0.6) (layer "F.Cu") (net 6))
 (segment (start 88.265 61.595) (end 95.115 61.595) (width 0.6) (layer "F.Cu") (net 6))
 (segment (start 123.17 58.03) (end 123.4 58.03) (width 0.6) (layer "F.Cu") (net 28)))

